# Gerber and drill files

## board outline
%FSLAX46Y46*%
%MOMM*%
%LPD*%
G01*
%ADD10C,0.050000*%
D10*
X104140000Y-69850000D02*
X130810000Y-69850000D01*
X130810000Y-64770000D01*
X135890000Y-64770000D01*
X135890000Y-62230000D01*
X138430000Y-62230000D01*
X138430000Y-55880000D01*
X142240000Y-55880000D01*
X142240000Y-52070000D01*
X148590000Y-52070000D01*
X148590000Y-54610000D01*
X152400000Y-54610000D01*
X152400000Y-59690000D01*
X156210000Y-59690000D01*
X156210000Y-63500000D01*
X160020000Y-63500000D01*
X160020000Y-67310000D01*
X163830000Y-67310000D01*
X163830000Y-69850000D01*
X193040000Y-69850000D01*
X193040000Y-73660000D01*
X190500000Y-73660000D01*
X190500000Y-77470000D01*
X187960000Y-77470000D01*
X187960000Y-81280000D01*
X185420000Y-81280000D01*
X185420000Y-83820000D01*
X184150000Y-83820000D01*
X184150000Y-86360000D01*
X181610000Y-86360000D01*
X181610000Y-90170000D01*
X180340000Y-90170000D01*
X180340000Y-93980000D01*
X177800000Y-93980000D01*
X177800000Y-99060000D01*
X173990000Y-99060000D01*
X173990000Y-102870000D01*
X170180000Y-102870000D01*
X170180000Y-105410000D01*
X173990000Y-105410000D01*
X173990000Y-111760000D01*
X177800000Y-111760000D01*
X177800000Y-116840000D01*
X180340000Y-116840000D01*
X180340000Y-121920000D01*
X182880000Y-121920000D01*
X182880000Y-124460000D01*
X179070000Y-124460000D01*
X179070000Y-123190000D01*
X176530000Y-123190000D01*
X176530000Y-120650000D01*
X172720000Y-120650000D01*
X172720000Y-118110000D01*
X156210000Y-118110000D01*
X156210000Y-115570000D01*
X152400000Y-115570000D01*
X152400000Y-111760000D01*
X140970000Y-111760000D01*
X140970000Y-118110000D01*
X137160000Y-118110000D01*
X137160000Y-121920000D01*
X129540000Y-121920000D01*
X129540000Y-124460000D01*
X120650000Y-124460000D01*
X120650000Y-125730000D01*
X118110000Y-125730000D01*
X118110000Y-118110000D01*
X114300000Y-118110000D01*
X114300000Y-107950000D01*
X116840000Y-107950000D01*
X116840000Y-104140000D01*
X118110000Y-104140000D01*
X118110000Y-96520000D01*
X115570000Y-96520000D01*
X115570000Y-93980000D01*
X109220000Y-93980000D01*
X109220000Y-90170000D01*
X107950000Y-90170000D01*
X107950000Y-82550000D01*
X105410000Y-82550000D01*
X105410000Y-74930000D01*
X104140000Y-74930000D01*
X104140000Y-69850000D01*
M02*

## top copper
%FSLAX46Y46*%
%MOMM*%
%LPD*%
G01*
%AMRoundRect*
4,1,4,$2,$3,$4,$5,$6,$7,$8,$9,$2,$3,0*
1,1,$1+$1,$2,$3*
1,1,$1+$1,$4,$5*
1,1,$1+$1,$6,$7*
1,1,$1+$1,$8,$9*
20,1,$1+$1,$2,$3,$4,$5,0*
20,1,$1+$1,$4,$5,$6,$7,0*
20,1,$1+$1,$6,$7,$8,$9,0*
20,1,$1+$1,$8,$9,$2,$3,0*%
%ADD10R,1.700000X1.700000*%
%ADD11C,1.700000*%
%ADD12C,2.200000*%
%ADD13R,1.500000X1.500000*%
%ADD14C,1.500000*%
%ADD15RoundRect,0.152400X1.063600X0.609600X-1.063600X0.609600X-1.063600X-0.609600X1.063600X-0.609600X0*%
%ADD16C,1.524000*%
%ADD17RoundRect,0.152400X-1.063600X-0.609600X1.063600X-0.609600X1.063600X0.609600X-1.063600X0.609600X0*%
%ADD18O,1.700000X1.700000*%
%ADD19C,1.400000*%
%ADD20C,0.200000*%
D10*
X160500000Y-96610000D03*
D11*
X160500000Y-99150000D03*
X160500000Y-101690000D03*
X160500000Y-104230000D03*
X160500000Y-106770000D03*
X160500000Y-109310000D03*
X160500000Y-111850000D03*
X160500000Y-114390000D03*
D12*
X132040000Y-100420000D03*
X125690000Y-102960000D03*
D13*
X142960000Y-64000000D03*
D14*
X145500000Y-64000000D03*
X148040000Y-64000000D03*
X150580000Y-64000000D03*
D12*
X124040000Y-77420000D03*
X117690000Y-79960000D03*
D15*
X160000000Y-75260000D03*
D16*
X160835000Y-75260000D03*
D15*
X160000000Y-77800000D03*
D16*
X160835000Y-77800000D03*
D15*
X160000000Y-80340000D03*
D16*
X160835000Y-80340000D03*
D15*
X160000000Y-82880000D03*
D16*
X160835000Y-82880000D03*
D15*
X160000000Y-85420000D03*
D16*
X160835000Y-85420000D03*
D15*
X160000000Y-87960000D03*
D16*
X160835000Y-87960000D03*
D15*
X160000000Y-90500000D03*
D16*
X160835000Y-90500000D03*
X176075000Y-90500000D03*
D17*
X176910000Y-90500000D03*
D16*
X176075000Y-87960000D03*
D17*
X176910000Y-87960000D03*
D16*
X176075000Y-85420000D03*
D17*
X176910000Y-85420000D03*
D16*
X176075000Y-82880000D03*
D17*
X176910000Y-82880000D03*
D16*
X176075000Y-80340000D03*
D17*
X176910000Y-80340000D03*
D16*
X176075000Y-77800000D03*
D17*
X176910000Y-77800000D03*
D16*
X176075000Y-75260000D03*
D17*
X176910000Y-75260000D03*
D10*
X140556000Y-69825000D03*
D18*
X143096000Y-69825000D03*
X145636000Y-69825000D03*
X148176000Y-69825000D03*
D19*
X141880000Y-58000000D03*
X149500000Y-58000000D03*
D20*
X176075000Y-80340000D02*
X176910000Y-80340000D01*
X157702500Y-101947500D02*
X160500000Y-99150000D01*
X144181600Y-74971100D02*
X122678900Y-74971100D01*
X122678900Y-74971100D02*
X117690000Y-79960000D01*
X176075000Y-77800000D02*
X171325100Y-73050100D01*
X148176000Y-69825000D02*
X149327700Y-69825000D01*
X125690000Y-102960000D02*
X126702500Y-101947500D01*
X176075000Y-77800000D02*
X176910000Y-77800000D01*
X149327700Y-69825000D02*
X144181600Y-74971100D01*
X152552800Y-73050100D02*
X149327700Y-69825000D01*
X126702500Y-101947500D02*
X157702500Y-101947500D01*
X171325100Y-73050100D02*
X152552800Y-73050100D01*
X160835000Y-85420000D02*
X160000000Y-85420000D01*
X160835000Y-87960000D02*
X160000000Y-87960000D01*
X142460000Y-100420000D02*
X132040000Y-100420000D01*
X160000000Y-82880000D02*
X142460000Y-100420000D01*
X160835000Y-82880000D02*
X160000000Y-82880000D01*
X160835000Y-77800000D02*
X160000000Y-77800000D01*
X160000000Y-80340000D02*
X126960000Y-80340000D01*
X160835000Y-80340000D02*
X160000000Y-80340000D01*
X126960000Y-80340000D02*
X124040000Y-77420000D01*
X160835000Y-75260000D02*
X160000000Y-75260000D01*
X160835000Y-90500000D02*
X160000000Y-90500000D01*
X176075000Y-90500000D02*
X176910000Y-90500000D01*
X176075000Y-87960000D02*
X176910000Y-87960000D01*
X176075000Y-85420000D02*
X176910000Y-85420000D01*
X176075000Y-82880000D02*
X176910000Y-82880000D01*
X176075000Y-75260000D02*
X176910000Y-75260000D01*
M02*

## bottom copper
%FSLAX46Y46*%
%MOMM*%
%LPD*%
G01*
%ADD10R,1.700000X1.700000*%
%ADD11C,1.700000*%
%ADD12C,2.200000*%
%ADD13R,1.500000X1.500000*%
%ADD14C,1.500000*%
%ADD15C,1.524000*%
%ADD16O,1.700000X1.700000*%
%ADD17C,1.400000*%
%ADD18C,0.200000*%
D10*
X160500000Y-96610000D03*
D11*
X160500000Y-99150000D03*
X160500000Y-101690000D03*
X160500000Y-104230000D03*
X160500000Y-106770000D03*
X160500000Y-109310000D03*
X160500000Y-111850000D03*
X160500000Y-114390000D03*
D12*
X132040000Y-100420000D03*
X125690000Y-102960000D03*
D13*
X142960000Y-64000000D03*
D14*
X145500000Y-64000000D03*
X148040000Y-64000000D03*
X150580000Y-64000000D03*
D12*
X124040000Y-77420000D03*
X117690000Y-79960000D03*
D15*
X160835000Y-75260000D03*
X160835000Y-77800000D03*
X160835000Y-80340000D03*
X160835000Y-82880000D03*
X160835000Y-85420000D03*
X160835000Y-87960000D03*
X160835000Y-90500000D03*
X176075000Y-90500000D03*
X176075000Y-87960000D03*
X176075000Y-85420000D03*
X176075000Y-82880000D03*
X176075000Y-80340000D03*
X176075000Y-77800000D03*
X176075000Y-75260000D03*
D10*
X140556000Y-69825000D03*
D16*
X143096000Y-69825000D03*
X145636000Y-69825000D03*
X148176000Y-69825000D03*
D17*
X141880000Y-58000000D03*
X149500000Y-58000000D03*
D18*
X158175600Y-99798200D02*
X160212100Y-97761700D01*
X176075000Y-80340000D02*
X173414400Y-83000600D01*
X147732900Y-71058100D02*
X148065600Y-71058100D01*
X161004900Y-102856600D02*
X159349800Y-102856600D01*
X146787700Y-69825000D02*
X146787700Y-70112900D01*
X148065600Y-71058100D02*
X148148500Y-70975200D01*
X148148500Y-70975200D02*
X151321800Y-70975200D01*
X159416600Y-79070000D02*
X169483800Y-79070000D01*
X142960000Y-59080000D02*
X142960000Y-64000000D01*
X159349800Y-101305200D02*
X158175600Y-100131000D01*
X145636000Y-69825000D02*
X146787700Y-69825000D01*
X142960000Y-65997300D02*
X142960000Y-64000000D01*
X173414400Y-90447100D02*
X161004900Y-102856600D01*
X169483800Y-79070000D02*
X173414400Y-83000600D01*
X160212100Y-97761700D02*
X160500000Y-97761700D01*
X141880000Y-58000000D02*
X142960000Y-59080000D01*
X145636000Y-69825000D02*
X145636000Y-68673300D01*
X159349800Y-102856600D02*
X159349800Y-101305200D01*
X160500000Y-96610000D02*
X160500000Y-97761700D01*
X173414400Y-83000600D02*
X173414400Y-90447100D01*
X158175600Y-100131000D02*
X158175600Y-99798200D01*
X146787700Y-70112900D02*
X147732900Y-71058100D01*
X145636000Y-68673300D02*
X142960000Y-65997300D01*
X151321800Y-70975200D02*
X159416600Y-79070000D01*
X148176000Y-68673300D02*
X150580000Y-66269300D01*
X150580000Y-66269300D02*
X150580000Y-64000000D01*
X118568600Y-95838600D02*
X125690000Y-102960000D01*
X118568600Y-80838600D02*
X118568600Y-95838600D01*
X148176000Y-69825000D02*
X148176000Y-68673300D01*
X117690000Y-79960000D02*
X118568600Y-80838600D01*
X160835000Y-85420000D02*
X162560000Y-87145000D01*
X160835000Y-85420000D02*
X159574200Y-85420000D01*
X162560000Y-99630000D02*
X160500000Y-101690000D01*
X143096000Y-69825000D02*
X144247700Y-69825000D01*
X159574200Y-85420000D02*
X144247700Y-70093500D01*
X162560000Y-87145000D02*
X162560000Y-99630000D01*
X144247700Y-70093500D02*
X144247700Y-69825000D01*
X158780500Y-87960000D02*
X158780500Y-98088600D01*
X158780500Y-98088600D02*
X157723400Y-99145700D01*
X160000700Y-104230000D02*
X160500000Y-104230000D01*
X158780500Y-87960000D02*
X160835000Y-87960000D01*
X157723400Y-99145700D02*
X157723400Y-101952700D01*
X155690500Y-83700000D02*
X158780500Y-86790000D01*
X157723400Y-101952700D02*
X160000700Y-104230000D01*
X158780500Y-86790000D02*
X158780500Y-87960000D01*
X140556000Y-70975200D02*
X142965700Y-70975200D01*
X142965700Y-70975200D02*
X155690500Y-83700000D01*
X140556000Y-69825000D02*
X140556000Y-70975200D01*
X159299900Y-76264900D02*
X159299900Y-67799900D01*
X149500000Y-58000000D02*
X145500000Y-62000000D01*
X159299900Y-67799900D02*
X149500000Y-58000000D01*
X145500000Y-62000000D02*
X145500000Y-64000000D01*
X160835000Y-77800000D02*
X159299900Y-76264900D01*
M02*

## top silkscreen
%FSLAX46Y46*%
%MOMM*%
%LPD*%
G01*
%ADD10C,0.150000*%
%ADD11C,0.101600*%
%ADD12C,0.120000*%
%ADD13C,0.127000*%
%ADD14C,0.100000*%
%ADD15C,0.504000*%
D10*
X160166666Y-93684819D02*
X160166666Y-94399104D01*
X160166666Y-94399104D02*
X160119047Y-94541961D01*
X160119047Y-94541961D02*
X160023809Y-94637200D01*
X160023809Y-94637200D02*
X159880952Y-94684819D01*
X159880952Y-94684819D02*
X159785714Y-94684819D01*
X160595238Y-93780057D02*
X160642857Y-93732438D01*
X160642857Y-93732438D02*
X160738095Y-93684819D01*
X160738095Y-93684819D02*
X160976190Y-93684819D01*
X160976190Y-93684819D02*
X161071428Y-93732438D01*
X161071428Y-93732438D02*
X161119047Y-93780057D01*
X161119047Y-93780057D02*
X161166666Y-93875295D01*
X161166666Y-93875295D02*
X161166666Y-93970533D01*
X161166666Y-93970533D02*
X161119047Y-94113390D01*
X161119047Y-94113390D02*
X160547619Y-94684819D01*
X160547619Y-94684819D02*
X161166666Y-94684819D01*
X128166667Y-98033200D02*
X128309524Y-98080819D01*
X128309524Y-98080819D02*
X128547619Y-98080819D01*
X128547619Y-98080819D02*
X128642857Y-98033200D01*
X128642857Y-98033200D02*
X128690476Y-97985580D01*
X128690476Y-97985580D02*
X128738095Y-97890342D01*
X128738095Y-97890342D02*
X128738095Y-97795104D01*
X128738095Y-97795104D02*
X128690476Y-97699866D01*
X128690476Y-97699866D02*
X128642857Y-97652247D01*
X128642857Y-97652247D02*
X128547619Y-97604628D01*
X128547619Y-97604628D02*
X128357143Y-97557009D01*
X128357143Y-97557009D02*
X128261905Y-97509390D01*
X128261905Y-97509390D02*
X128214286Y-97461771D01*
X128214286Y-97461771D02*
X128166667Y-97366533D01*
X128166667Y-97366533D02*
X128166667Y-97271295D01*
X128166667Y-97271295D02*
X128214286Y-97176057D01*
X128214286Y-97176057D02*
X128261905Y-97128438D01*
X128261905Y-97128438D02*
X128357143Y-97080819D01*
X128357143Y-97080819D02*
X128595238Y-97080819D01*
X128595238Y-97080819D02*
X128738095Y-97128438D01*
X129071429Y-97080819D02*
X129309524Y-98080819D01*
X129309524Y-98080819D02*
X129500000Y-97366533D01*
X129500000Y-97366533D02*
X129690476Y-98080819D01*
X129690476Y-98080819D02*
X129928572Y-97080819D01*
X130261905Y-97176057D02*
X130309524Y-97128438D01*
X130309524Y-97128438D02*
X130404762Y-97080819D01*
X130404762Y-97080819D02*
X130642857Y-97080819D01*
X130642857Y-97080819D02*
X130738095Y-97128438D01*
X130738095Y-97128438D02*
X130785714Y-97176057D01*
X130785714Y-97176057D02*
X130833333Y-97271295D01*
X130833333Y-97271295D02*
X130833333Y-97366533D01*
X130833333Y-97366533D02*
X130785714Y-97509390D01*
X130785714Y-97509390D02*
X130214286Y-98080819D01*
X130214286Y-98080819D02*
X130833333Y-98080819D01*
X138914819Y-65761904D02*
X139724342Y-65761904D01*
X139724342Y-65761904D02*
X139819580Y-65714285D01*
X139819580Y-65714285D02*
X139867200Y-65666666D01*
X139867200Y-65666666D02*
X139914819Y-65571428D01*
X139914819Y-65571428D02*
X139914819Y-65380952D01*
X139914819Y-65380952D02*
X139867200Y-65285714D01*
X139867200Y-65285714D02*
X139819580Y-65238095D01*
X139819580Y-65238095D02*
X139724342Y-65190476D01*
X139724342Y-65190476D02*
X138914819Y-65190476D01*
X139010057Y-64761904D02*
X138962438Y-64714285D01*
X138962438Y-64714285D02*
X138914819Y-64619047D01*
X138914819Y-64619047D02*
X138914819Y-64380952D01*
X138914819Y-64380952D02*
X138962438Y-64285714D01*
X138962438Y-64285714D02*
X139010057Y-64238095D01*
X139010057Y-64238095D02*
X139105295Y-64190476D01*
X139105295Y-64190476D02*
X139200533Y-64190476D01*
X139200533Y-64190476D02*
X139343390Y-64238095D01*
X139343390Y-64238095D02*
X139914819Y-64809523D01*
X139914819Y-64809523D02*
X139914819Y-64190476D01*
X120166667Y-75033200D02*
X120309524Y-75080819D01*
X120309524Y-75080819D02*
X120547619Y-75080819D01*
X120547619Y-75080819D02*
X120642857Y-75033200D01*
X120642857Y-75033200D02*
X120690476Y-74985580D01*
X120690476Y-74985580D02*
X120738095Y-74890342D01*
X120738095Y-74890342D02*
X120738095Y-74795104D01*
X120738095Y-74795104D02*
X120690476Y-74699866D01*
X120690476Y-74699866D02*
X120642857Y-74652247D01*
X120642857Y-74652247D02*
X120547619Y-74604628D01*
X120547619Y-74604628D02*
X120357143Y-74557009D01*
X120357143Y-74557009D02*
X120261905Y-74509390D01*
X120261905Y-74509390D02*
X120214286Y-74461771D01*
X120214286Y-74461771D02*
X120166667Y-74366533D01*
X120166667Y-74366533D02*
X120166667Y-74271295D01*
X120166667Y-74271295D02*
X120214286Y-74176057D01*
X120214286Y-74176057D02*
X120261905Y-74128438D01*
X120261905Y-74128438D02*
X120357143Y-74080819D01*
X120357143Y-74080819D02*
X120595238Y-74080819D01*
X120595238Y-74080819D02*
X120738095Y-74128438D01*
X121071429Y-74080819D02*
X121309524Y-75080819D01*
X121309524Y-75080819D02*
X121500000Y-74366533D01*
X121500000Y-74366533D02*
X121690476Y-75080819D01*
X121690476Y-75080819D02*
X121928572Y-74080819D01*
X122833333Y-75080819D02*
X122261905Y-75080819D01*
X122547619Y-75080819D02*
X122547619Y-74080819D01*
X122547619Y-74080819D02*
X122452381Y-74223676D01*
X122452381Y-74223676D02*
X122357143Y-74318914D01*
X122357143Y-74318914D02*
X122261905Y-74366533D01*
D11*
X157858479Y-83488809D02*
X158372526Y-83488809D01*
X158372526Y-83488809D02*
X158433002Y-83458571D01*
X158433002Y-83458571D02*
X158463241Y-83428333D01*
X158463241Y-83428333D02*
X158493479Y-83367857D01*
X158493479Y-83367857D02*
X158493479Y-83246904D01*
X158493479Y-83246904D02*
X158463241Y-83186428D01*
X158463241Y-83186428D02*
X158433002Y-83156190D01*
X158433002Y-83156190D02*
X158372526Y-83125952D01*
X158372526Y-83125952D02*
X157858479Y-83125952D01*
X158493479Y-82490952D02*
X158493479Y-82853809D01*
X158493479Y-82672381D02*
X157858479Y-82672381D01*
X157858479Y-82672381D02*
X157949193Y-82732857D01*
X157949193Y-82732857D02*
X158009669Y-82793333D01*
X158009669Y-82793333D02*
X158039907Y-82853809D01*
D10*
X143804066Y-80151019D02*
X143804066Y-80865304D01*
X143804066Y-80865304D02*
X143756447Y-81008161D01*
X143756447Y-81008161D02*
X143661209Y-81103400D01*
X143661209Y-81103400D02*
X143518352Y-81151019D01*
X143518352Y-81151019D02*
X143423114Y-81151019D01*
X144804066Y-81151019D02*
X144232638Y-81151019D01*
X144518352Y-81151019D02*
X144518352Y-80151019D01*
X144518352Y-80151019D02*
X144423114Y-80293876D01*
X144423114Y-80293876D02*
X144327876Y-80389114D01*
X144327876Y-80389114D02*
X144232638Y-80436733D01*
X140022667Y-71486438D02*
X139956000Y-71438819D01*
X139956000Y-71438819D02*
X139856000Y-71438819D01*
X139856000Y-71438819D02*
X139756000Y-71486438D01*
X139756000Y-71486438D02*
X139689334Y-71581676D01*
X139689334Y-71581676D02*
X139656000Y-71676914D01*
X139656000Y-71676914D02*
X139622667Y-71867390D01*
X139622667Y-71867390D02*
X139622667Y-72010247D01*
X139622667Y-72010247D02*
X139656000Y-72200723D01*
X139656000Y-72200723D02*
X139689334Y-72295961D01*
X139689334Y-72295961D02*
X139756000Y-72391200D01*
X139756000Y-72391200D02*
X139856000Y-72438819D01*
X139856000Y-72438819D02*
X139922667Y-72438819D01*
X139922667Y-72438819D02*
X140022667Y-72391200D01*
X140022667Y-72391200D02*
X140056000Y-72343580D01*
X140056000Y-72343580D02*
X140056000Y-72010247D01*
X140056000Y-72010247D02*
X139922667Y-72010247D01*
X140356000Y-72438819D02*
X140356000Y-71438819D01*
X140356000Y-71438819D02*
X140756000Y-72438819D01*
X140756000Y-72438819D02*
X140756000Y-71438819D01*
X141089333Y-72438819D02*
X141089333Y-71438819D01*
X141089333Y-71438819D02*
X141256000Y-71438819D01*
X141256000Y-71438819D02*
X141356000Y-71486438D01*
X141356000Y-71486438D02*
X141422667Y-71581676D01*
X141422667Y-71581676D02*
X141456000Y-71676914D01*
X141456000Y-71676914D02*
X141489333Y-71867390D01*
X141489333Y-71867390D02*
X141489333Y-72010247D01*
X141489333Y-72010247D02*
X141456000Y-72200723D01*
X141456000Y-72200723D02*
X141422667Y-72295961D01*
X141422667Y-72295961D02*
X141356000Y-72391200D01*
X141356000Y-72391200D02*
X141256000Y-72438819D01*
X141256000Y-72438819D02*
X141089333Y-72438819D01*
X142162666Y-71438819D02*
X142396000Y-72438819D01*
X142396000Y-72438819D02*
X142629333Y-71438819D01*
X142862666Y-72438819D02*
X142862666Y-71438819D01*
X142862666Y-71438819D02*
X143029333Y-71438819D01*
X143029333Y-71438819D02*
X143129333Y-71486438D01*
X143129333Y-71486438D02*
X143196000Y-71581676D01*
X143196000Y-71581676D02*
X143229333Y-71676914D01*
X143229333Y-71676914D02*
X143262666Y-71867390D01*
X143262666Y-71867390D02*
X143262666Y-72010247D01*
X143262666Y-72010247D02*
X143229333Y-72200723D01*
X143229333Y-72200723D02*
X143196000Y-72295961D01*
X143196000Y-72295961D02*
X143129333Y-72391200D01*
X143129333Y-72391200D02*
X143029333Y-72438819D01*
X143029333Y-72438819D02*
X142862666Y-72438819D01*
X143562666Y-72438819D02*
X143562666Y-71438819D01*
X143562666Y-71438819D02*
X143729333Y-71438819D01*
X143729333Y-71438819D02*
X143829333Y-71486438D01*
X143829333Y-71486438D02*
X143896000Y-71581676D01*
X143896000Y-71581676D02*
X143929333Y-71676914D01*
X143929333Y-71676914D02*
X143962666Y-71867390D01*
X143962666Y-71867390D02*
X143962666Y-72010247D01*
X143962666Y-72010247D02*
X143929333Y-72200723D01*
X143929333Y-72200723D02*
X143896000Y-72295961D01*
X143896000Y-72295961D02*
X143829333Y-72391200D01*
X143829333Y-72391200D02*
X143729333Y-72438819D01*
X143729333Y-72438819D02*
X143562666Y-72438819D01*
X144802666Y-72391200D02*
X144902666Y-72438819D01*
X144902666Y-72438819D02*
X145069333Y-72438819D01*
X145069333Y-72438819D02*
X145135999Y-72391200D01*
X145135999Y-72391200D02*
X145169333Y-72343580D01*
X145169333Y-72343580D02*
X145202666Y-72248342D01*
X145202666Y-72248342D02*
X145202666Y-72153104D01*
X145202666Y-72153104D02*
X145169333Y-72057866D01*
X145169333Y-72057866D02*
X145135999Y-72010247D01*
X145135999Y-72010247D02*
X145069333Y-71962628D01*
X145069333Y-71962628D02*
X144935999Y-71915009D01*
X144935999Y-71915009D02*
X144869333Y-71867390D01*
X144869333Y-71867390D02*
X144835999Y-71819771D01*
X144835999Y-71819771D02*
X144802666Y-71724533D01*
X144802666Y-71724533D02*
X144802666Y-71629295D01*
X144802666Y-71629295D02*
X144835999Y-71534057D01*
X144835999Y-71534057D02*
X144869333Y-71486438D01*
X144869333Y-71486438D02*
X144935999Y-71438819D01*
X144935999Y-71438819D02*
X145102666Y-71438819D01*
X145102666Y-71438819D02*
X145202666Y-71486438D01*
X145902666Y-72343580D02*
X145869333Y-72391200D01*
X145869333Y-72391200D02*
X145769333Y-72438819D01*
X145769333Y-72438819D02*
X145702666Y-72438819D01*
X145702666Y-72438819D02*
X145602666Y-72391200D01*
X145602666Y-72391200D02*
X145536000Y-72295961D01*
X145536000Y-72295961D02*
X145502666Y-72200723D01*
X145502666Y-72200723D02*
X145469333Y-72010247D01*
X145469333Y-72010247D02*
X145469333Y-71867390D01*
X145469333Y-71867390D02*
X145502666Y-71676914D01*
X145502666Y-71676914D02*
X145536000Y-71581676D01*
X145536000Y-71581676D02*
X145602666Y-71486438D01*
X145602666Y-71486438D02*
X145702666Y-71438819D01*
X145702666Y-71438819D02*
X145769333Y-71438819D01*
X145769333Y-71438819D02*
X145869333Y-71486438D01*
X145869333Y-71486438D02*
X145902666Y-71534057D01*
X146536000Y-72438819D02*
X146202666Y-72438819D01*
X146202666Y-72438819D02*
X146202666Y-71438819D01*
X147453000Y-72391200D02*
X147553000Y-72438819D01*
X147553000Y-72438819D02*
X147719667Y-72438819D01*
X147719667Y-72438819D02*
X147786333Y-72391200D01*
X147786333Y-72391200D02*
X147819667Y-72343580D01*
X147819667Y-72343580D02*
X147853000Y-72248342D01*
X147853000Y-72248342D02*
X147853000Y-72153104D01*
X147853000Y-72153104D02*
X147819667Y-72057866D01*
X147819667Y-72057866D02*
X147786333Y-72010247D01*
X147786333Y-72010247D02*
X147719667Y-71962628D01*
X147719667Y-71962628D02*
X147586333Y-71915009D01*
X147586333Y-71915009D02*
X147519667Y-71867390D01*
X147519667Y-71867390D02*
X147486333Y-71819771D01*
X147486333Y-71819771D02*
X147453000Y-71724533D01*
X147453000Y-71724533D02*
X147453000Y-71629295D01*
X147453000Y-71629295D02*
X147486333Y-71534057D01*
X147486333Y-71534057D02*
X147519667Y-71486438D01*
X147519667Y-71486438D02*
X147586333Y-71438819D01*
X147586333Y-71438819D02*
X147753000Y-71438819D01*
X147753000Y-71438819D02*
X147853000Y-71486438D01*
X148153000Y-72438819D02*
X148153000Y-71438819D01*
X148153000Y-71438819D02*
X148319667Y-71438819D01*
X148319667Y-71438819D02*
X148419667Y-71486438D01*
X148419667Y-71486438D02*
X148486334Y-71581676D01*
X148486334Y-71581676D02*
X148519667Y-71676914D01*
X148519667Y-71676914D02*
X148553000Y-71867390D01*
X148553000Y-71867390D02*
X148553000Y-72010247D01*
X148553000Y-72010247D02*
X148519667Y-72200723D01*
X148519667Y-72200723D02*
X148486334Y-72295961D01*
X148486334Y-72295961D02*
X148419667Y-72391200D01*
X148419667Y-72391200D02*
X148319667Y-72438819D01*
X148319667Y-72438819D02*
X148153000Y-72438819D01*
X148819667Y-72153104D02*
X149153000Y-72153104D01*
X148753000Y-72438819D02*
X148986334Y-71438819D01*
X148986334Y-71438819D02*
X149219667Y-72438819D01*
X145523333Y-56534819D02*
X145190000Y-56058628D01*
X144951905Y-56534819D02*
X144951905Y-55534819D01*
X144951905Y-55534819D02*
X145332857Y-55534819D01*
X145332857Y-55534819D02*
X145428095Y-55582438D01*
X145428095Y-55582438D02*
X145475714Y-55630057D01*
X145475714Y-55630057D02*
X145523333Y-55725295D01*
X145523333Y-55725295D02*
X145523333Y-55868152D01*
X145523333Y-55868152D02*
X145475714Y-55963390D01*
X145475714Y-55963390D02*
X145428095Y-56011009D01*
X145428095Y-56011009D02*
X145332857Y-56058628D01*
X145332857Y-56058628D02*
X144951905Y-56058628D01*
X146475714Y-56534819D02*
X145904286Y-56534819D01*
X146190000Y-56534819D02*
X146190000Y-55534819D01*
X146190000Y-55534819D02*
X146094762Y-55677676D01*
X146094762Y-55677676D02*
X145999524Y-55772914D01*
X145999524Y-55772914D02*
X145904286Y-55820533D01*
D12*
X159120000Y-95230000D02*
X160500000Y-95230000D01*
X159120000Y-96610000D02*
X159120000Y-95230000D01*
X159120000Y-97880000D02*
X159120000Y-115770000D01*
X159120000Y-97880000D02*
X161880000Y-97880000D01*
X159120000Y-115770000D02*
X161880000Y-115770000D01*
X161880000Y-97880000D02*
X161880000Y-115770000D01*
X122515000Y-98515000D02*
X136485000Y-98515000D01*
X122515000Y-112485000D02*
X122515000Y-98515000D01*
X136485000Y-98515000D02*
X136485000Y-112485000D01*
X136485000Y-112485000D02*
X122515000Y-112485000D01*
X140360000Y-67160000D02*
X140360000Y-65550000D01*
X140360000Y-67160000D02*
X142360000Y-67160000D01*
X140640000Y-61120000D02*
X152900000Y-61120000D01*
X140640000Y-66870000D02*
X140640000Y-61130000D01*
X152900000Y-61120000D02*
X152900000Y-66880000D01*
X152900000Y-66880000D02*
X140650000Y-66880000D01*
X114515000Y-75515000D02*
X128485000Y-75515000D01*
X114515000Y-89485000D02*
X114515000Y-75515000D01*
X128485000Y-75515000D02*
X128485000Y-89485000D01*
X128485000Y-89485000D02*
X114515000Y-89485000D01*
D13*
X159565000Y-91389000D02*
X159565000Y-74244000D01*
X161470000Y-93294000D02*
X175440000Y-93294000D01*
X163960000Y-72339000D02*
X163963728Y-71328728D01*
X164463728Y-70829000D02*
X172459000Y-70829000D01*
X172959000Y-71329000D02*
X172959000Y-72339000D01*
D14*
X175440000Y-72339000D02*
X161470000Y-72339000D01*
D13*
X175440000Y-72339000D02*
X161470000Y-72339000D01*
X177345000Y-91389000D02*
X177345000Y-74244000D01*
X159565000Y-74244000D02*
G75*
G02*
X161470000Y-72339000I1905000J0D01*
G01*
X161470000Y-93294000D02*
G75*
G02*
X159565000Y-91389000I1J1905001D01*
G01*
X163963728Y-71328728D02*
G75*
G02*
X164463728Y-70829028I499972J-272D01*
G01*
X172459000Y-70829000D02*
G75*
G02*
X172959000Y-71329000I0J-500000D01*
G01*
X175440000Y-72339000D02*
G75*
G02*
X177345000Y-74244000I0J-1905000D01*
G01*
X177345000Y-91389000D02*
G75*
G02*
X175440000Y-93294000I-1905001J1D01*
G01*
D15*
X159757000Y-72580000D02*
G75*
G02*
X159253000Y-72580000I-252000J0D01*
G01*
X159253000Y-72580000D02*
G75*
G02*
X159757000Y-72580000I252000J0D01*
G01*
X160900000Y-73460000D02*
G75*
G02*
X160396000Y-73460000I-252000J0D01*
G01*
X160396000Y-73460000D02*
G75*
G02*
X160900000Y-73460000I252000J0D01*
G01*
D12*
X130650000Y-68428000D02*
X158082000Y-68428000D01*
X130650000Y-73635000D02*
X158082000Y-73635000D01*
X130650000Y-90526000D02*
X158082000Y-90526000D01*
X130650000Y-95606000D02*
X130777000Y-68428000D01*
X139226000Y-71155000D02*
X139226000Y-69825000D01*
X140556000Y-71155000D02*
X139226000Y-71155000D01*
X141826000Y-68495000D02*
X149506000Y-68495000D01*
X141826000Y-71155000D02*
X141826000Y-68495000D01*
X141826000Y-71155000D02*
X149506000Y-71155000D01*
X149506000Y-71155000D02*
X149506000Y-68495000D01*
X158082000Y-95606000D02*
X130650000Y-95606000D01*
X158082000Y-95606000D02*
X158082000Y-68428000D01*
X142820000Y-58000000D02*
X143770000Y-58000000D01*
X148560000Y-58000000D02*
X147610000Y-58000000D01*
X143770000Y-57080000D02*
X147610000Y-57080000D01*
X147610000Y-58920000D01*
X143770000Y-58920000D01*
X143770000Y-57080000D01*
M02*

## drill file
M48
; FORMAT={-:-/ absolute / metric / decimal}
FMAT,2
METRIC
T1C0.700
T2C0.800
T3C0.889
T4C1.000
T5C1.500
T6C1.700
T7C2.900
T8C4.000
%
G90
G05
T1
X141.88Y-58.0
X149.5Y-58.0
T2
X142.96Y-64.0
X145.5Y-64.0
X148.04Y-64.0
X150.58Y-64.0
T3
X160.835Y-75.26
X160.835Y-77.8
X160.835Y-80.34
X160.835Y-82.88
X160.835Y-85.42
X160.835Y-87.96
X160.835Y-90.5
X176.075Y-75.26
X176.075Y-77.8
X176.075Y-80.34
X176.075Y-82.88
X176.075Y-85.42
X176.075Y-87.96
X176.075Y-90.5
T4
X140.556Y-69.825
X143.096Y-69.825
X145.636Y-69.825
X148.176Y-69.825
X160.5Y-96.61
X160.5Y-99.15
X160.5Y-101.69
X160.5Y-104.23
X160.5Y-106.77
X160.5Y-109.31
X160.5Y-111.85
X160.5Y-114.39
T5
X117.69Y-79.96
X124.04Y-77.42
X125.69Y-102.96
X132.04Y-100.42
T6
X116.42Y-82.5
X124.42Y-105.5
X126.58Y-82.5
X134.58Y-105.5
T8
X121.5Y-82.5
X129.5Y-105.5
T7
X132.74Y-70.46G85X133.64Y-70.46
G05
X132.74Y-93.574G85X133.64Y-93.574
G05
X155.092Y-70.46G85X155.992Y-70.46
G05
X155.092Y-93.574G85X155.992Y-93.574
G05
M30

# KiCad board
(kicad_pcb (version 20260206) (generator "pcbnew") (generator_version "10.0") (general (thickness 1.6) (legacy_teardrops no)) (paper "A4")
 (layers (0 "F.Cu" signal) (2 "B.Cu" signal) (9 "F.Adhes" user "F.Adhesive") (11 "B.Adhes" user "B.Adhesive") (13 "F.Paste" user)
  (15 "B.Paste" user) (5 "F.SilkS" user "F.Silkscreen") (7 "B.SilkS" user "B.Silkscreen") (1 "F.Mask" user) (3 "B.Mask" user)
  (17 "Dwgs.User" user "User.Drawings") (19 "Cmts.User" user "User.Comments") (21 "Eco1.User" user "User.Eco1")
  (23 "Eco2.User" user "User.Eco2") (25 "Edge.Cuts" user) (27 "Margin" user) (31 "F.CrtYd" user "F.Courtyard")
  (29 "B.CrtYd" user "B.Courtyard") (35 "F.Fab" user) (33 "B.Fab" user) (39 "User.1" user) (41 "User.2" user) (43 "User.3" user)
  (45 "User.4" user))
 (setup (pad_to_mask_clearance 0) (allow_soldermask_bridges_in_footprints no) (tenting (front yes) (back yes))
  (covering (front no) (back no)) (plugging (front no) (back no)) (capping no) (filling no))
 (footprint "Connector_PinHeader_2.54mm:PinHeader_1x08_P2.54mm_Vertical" (layer "F.Cu") (at 160.5 96.61)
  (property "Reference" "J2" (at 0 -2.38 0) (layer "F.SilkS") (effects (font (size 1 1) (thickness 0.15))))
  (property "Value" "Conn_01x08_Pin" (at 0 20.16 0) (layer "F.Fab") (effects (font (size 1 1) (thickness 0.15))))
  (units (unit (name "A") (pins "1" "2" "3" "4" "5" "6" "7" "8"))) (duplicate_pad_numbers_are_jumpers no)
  (fp_line (start -1.38 -1.38) (end 0 -1.38) (stroke (width 0.12) (type solid)) (layer "F.SilkS"))
  (fp_line (start -1.38 0) (end -1.38 -1.38) (stroke (width 0.12) (type solid)) (layer "F.SilkS"))
  (fp_line (start -1.38 1.27) (end -1.38 19.16) (stroke (width 0.12) (type solid)) (layer "F.SilkS"))
  (fp_line (start -1.38 1.27) (end 1.38 1.27) (stroke (width 0.12) (type solid)) (layer "F.SilkS"))
  (fp_line (start -1.38 19.16) (end 1.38 19.16) (stroke (width 0.12) (type solid)) (layer "F.SilkS"))
  (fp_line (start 1.38 1.27) (end 1.38 19.16) (stroke (width 0.12) (type solid)) (layer "F.SilkS"))
  (pad "1" thru_hole rect (at 0 0) (size 1.7 1.7) (drill 1) (layers "*.Cu" "*.Mask") (remove_unused_layers no) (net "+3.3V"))
  (pad "2" thru_hole circle (at 0 2.54) (size 1.7 1.7) (drill 1) (layers "*.Cu" "*.Mask") (remove_unused_layers no) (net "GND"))
  (pad "3" thru_hole circle (at 0 5.08) (size 1.7 1.7) (drill 1) (layers "*.Cu" "*.Mask") (remove_unused_layers no) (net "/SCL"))
  (pad "4" thru_hole circle (at 0 7.62) (size 1.7 1.7) (drill 1) (layers "*.Cu" "*.Mask") (remove_unused_layers no) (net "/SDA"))
  (pad "5" thru_hole circle (at 0 10.16) (size 1.7 1.7) (drill 1) (layers "*.Cu" "*.Mask") (remove_unused_layers no)
   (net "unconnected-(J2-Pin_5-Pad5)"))
  (pad "6" thru_hole circle (at 0 12.7) (size 1.7 1.7) (drill 1) (layers "*.Cu" "*.Mask") (remove_unused_layers no)
   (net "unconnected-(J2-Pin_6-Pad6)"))
  (pad "7" thru_hole circle (at 0 15.24) (size 1.7 1.7) (drill 1) (layers "*.Cu" "*.Mask") (remove_unused_layers no)
   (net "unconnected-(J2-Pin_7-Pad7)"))
  (pad "8" thru_hole circle (at 0 17.78) (size 1.7 1.7) (drill 1) (layers "*.Cu" "*.Mask") (remove_unused_layers no)
   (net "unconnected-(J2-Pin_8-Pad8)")))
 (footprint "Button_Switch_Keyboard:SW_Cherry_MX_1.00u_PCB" (layer "F.Cu") (at 132.04 100.42)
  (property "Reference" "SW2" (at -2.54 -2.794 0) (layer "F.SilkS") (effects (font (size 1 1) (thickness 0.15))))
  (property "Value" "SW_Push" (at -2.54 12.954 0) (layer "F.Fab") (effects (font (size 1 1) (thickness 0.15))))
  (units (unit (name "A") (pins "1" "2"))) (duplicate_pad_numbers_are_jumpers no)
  (fp_line (start -9.525 -1.905) (end 4.445 -1.905) (stroke (width 0.12) (type solid)) (layer "F.SilkS"))
  (fp_line (start -9.525 12.065) (end -9.525 -1.905) (stroke (width 0.12) (type solid)) (layer "F.SilkS"))
  (fp_line (start 4.445 -1.905) (end 4.445 12.065) (stroke (width 0.12) (type solid)) (layer "F.SilkS"))
  (fp_line (start 4.445 12.065) (end -9.525 12.065) (stroke (width 0.12) (type solid)) (layer "F.SilkS"))
  (pad "" np_thru_hole circle (at -7.62 5.08) (size 1.7 1.7) (drill 1.7) (layers "*.Cu" "*.Mask"))
  (pad "" np_thru_hole circle (at -2.54 5.08) (size 4 4) (drill 4) (layers "*.Cu" "*.Mask"))
  (pad "" np_thru_hole circle (at 2.54 5.08) (size 1.7 1.7) (drill 1.7) (layers "*.Cu" "*.Mask"))
  (pad "1" thru_hole circle (at 0 0) (size 2.2 2.2) (drill 1.5) (layers "*.Cu" "*.Mask") (remove_unused_layers no) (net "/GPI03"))
  (pad "2" thru_hole circle (at -6.35 2.54) (size 2.2 2.2) (drill 1.5) (layers "*.Cu" "*.Mask") (remove_unused_layers no) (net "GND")))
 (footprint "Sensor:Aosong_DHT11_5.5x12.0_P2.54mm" (layer "F.Cu") (at 142.96 64 90)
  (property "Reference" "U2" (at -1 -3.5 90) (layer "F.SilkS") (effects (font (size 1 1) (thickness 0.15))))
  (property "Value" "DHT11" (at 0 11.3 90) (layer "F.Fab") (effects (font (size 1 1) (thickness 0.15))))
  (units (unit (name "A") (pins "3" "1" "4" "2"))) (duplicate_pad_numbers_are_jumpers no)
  (fp_line (start -3.16 -2.6) (end -1.55 -2.6) (stroke (width 0.12) (type solid)) (layer "F.SilkS"))
  (fp_line (start -3.16 -2.6) (end -3.16 -0.6) (stroke (width 0.12) (type solid)) (layer "F.SilkS"))
  (fp_line (start 2.88 -2.32) (end 2.88 9.94) (stroke (width 0.12) (type solid)) (layer "F.SilkS"))
  (fp_line (start -2.87 -2.32) (end 2.87 -2.32) (stroke (width 0.12) (type solid)) (layer "F.SilkS"))
  (fp_line (start 2.88 9.94) (end -2.88 9.94) (stroke (width 0.12) (type solid)) (layer "F.SilkS"))
  (fp_line (start -2.88 9.94) (end -2.88 -2.31) (stroke (width 0.12) (type solid)) (layer "F.SilkS"))
  (pad "1" thru_hole rect (at 0 0 90) (size 1.5 1.5) (drill 0.8) (layers "*.Cu" "*.Mask") (remove_unused_layers no) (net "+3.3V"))
  (pad "2" thru_hole circle (at 0 2.54 90) (size 1.5 1.5) (drill 0.8) (layers "*.Cu" "*.Mask") (remove_unused_layers no) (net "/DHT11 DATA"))
  (pad "3" thru_hole circle (at 0 5.08 90) (size 1.5 1.5) (drill 0.8) (layers "*.Cu" "*.Mask") (remove_unused_layers no)
   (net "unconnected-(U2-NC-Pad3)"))
  (pad "4" thru_hole circle (at 0 7.62 90) (size 1.5 1.5) (drill 0.8) (layers "*.Cu" "*.Mask") (remove_unused_layers no) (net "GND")))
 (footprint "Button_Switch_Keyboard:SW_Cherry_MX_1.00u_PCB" (layer "F.Cu") (at 124.04 77.42)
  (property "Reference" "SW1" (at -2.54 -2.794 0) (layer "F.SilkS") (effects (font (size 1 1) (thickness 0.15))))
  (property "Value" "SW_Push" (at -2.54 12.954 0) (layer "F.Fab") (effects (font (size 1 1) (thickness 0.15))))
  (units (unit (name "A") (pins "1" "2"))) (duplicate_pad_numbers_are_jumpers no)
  (fp_line (start -9.525 -1.905) (end 4.445 -1.905) (stroke (width 0.12) (type solid)) (layer "F.SilkS"))
  (fp_line (start -9.525 12.065) (end -9.525 -1.905) (stroke (width 0.12) (type solid)) (layer "F.SilkS"))
  (fp_line (start 4.445 -1.905) (end 4.445 12.065) (stroke (width 0.12) (type solid)) (layer "F.SilkS"))
  (fp_line (start 4.445 12.065) (end -9.525 12.065) (stroke (width 0.12) (type solid)) (layer "F.SilkS"))
  (pad "" np_thru_hole circle (at -7.62 5.08) (size 1.7 1.7) (drill 1.7) (layers "*.Cu" "*.Mask"))
  (pad "" np_thru_hole circle (at -2.54 5.08) (size 4 4) (drill 4) (layers "*.Cu" "*.Mask"))
  (pad "" np_thru_hole circle (at 2.54 5.08) (size 1.7 1.7) (drill 1.7) (layers "*.Cu" "*.Mask"))
  (pad "1" thru_hole circle (at 0 0) (size 2.2 2.2) (drill 1.5) (layers "*.Cu" "*.Mask") (remove_unused_layers no) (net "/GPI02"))
  (pad "2" thru_hole circle (at -6.35 2.54) (size 2.2 2.2) (drill 1.5) (layers "*.Cu" "*.Mask") (remove_unused_layers no) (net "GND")))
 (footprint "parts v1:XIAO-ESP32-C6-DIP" (layer "F.Cu") (at 168.455 82.88 90)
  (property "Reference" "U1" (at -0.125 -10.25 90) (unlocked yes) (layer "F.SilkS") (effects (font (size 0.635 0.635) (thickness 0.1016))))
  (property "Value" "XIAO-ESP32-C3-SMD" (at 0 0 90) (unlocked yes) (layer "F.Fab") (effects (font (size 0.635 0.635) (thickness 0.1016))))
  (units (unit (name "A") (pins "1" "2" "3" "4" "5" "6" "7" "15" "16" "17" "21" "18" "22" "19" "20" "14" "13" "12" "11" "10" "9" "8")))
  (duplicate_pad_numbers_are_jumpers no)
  (fp_line (start -8.509 -8.89) (end 8.636 -8.89) (stroke (width 0.127) (type solid)) (layer "F.SilkS"))
  (fp_line (start -10.414 -6.985) (end -10.414 6.985) (stroke (width 0.127) (type solid)) (layer "F.SilkS"))
  (fp_line (start 10.541 -4.495) (end 11.551272 -4.491272) (stroke (width 0.127) (type solid)) (layer "F.SilkS"))
  (fp_line (start 12.051 -3.991272) (end 12.051 4.004) (stroke (width 0.127) (type solid)) (layer "F.SilkS"))
  (fp_line (start 11.551 4.504) (end 10.541 4.504) (stroke (width 0.127) (type solid)) (layer "F.SilkS"))
  (fp_line (start 10.541 6.985) (end 10.541 -6.985) (stroke (width 0.1) (type solid)) (layer "F.SilkS"))
  (fp_line (start 10.541 6.985) (end 10.541 -6.985) (stroke (width 0.127) (type solid)) (layer "F.SilkS"))
  (fp_line (start -8.509 8.89) (end 8.636 8.89) (stroke (width 0.127) (type solid)) (layer "F.SilkS"))
  (fp_arc (start 8.636 -8.89) (mid 9.983038 -8.332038) (end 10.541 -6.985) (stroke (width 0.127) (type solid)) (layer "F.SilkS"))
  (fp_arc (start -10.414 -6.985) (mid -9.856038 -8.332038) (end -8.509 -8.89) (stroke (width 0.127) (type solid)) (layer "F.SilkS"))
  (fp_arc (start 11.551272 -4.491272) (mid 11.904644 -4.344724) (end 12.051 -3.991272) (stroke (width 0.127) (type default))
   (layer "F.SilkS"))
  (fp_arc (start 12.051 4.004) (mid 11.904553 4.357553) (end 11.551 4.504) (stroke (width 0.127) (type default)) (layer "F.SilkS"))
  (fp_arc (start 10.541 6.985) (mid 9.983038 8.332038) (end 8.636 8.89) (stroke (width 0.127) (type solid)) (layer "F.SilkS"))
  (fp_arc (start -8.509 8.89) (mid -9.856038 8.332038) (end -10.414 6.985) (stroke (width 0.127) (type solid)) (layer "F.SilkS"))
  (fp_circle (center 10.3 -8.95) (end 10.554 -8.95) (stroke (width 0.5) (type solid)) (fill yes) (layer "F.SilkS"))
  (fp_circle (center 9.42 -7.807) (end 9.674 -7.807) (stroke (width 0.5) (type solid)) (fill yes) (layer "F.SilkS"))
  (pad "1" smd roundrect (at 7.62 -8.455 180) (size 2.432 1.524) (layers "F.Cu" "F.Mask") (roundrect_rratio 0.1)
   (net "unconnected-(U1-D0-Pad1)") (thermal_bridge_angle 45))
  (pad "1" thru_hole circle (at 7.62 -7.62 180) (size 1.524 1.524) (drill 0.889) (layers "*.Cu" "*.Mask") (remove_unused_layers no)
   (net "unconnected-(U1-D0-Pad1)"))
  (pad "2" smd roundrect (at 5.08 -8.455 180) (size 2.432 1.524) (layers "F.Cu" "F.Mask") (roundrect_rratio 0.1) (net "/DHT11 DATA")
   (thermal_bridge_angle 45))
  (pad "2" thru_hole circle (at 5.08 -7.62 180) (size 1.524 1.524) (drill 0.889) (layers "*.Cu" "*.Mask") (remove_unused_layers no)
   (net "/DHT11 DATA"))
  (pad "3" smd roundrect (at 2.54 -8.455 180) (size 2.432 1.524) (layers "F.Cu" "F.Mask") (roundrect_rratio 0.1) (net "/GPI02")
   (thermal_bridge_angle 45))
  (pad "3" thru_hole circle (at 2.54 -7.62 180) (size 1.524 1.524) (drill 0.889) (layers "*.Cu" "*.Mask") (remove_unused_layers no)
   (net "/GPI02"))
  (pad "4" smd roundrect (at 0 -8.455 180) (size 2.432 1.524) (layers "F.Cu" "F.Mask") (roundrect_rratio 0.1) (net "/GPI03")
   (thermal_bridge_angle 45))
  (pad "4" thru_hole circle (at 0 -7.62 180) (size 1.524 1.524) (drill 0.889) (layers "*.Cu" "*.Mask") (remove_unused_layers no)
   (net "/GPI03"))
  (pad "5" smd roundrect (at -2.54 -8.455 180) (size 2.432 1.524) (layers "F.Cu" "F.Mask") (roundrect_rratio 0.1) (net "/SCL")
   (thermal_bridge_angle 45))
  (pad "5" thru_hole circle (at -2.54 -7.62 180) (size 1.524 1.524) (drill 0.889) (layers "*.Cu" "*.Mask") (remove_unused_layers no)
   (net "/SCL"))
  (pad "6" smd roundrect (at -5.08 -8.455 180) (size 2.432 1.524) (layers "F.Cu" "F.Mask") (roundrect_rratio 0.1) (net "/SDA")
   (thermal_bridge_angle 45))
  (pad "6" thru_hole circle (at -5.08 -7.62 180) (size 1.524 1.524) (drill 0.889) (layers "*.Cu" "*.Mask") (remove_unused_layers no)
   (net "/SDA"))
  (pad "7" smd roundrect (at -7.62 -8.455 180) (size 2.432 1.524) (layers "F.Cu" "F.Mask") (roundrect_rratio 0.1)
   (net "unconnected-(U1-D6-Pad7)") (thermal_bridge_angle 45))
  (pad "7" thru_hole circle (at -7.62 -7.62 180) (size 1.524 1.524) (drill 0.889) (layers "*.Cu" "*.Mask") (remove_unused_layers no)
   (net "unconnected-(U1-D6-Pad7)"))
  (pad "8" thru_hole circle (at -7.62 7.62) (size 1.524 1.524) (drill 0.889) (layers "*.Cu" "*.Mask") (remove_unused_layers no)
   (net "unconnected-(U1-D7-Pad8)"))
  (pad "8" smd roundrect (at -7.62 8.455) (size 2.432 1.524) (layers "F.Cu" "F.Mask") (roundrect_rratio 0.1)
   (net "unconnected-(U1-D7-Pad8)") (thermal_bridge_angle 45))
  (pad "9" thru_hole circle (at -5.08 7.62) (size 1.524 1.524) (drill 0.889) (layers "*.Cu" "*.Mask") (remove_unused_layers no)
   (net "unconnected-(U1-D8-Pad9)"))
  (pad "9" smd roundrect (at -5.08 8.455) (size 2.432 1.524) (layers "F.Cu" "F.Mask") (roundrect_rratio 0.1)
   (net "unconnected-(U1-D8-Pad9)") (thermal_bridge_angle 45))
  (pad "10" thru_hole circle (at -2.54 7.62) (size 1.524 1.524) (drill 0.889) (layers "*.Cu" "*.Mask") (remove_unused_layers no)
   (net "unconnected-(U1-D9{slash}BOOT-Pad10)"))
  (pad "10" smd roundrect (at -2.54 8.455) (size 2.432 1.524) (layers "F.Cu" "F.Mask") (roundrect_rratio 0.1)
   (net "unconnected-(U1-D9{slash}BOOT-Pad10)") (thermal_bridge_angle 45))
  (pad "11" thru_hole circle (at 0 7.62) (size 1.524 1.524) (drill 0.889) (layers "*.Cu" "*.Mask") (remove_unused_layers no)
   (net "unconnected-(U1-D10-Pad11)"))
  (pad "11" smd roundrect (at 0 8.455) (size 2.432 1.524) (layers "F.Cu" "F.Mask") (roundrect_rratio 0.1) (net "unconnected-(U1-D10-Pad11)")
   (thermal_bridge_angle 45))
  (pad "12" thru_hole circle (at 2.54 7.62) (size 1.524 1.524) (drill 0.889) (layers "*.Cu" "*.Mask") (remove_unused_layers no)
   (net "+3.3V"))
  (pad "12" smd roundrect (at 2.54 8.455) (size 2.432 1.524) (layers "F.Cu" "F.Mask") (roundrect_rratio 0.1) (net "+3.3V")
   (thermal_bridge_angle 45))
  (pad "13" thru_hole circle (at 5.08 7.62) (size 1.524 1.524) (drill 0.889) (layers "*.Cu" "*.Mask") (remove_unused_layers no) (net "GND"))
  (pad "13" smd roundrect (at 5.08 8.455) (size 2.432 1.524) (layers "F.Cu" "F.Mask") (roundrect_rratio 0.1) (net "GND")
   (thermal_bridge_angle 45))
  (pad "14" thru_hole circle (at 7.62 7.62) (size 1.524 1.524) (drill 0.889) (layers "*.Cu" "*.Mask") (remove_unused_layers no) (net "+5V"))
  (pad "14" smd roundrect (at 7.62 8.455) (size 2.432 1.524) (layers "F.Cu" "F.Mask") (roundrect_rratio 0.1) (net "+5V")
   (thermal_bridge_angle 45)))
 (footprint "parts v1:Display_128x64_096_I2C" (layer "F.Cu") (at 144.366 69.825)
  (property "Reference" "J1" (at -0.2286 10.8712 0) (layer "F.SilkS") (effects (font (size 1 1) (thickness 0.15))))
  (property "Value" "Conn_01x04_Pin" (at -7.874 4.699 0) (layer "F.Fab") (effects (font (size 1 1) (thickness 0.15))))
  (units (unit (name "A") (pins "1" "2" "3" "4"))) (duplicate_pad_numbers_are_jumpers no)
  (fp_line (start -13.716 -1.397) (end 13.716 -1.397) (stroke (width 0.12) (type solid)) (layer "F.SilkS"))
  (fp_line (start -13.716 3.81) (end 13.716 3.81) (stroke (width 0.12) (type solid)) (layer "F.SilkS"))
  (fp_line (start -13.716 20.701) (end 13.716 20.701) (stroke (width 0.12) (type solid)) (layer "F.SilkS"))
  (fp_line (start -13.716 25.781) (end -13.589 -1.397) (stroke (width 0.12) (type solid)) (layer "F.SilkS"))
  (fp_line (start -5.14 1.33) (end -5.14 0) (stroke (width 0.12) (type solid)) (layer "F.SilkS"))
  (fp_line (start -3.81 1.33) (end -5.14 1.33) (stroke (width 0.12) (type solid)) (layer "F.SilkS"))
  (fp_line (start -2.54 -1.33) (end 5.14 -1.33) (stroke (width 0.12) (type solid)) (layer "F.SilkS"))
  (fp_line (start -2.54 1.33) (end -2.54 -1.33) (stroke (width 0.12) (type solid)) (layer "F.SilkS"))
  (fp_line (start -2.54 1.33) (end 5.14 1.33) (stroke (width 0.12) (type solid)) (layer "F.SilkS"))
  (fp_line (start 5.14 1.33) (end 5.14 -1.33) (stroke (width 0.12) (type solid)) (layer "F.SilkS"))
  (fp_line (start 13.716 25.781) (end -13.716 25.781) (stroke (width 0.12) (type solid)) (layer "F.SilkS"))
  (fp_line (start 13.716 25.781) (end 13.716 -1.397) (stroke (width 0.12) (type solid)) (layer "F.SilkS"))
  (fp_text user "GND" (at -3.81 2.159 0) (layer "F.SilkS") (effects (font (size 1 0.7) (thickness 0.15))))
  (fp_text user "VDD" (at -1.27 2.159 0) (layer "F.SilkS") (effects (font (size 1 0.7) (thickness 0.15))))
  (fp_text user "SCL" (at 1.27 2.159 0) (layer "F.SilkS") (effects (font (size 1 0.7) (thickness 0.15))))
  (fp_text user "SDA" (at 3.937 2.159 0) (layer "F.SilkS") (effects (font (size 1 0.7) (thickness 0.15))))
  (pad "" np_thru_hole oval (at -11.176 0.635) (size 3.8 2.9) (drill oval 3.8 2.9) (layers "*.Cu" "*.Mask"))
  (pad "" np_thru_hole oval (at -11.176 23.749) (size 3.8 2.9) (drill oval 3.8 2.9) (layers "*.Cu" "*.Mask"))
  (pad "" np_thru_hole oval (at 11.176 0.635) (size 3.8 2.9) (drill oval 3.8 2.9) (layers "*.Cu" "*.Mask"))
  (pad "" np_thru_hole oval (at 11.176 23.749) (size 3.8 2.9) (drill oval 3.8 2.9) (layers "*.Cu" "*.Mask"))
  (pad "1" thru_hole rect (at -3.81 0 90) (size 1.7 1.7) (drill 1) (layers "*.Cu" "*.Mask") (remove_unused_layers no) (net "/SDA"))
  (pad "2" thru_hole oval (at -1.27 0 90) (size 1.7 1.7) (drill 1) (layers "*.Cu" "*.Mask") (remove_unused_layers no) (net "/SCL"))
  (pad "3" thru_hole oval (at 1.27 0 90) (size 1.7 1.7) (drill 1) (layers "*.Cu" "*.Mask") (remove_unused_layers no) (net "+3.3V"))
  (pad "4" thru_hole oval (at 3.81 0 90) (size 1.7 1.7) (drill 1) (layers "*.Cu" "*.Mask") (remove_unused_layers no) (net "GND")))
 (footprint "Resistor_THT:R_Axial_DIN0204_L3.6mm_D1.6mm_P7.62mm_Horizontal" (layer "F.Cu") (at 141.88 58)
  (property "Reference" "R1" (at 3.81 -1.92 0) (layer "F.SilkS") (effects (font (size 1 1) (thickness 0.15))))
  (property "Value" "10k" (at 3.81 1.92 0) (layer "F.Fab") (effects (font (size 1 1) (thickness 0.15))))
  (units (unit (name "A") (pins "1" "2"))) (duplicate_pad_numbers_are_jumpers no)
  (fp_line (start 0.94 0) (end 1.89 0) (stroke (width 0.12) (type solid)) (layer "F.SilkS"))
  (fp_line (start 6.68 0) (end 5.73 0) (stroke (width 0.12) (type solid)) (layer "F.SilkS"))
  (fp_rect (start 1.89 -0.92) (end 5.73 0.92) (stroke (width 0.12) (type solid)) (fill no) (layer "F.SilkS"))
  (pad "1" thru_hole circle (at 0 0) (size 1.4 1.4) (drill 0.7) (layers "*.Cu" "*.Mask") (remove_unused_layers no) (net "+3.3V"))
  (pad "2" thru_hole circle (at 7.62 0) (size 1.4 1.4) (drill 0.7) (layers "*.Cu" "*.Mask") (remove_unused_layers no) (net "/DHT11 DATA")))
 (gr_poly
  (pts (xy 104.14 69.85) (xy 130.81 69.85) (xy 130.81 64.77) (xy 135.89 64.77) (xy 135.89 62.23) (xy 138.43 62.23) (xy 138.43 55.88)
   (xy 142.24 55.88) (xy 142.24 52.07) (xy 148.59 52.07) (xy 148.59 54.61) (xy 152.4 54.61) (xy 152.4 59.69) (xy 156.21 59.69)
   (xy 156.21 63.5) (xy 160.02 63.5) (xy 160.02 67.31) (xy 163.83 67.31) (xy 163.83 69.85) (xy 193.04 69.85) (xy 193.04 73.66)
   (xy 190.5 73.66) (xy 190.5 77.47) (xy 187.96 77.47) (xy 187.96 81.28) (xy 185.42 81.28) (xy 185.42 83.82) (xy 184.15 83.82)
   (xy 184.15 86.36) (xy 181.61 86.36) (xy 181.61 90.17) (xy 180.34 90.17) (xy 180.34 93.98) (xy 177.8 93.98) (xy 177.8 99.06)
   (xy 173.99 99.06) (xy 173.99 102.87) (xy 170.18 102.87) (xy 170.18 105.41) (xy 173.99 105.41) (xy 173.99 111.76) (xy 177.8 111.76)
   (xy 177.8 116.84) (xy 180.34 116.84) (xy 180.34 121.92) (xy 182.88 121.92) (xy 182.88 124.46) (xy 179.07 124.46) (xy 179.07 123.19)
   (xy 176.53 123.19) (xy 176.53 120.65) (xy 172.72 120.65) (xy 172.72 118.11) (xy 156.21 118.11) (xy 156.21 115.57) (xy 152.4 115.57)
   (xy 152.4 111.76) (xy 140.97 111.76) (xy 140.97 118.11) (xy 137.16 118.11) (xy 137.16 121.92) (xy 129.54 121.92) (xy 129.54 124.46)
   (xy 120.65 124.46) (xy 120.65 125.73) (xy 118.11 125.73) (xy 118.11 118.11) (xy 114.3 118.11) (xy 114.3 107.95) (xy 116.84 107.95)
   (xy 116.84 104.14) (xy 118.11 104.14) (xy 118.11 96.52) (xy 115.57 96.52) (xy 115.57 93.98) (xy 109.22 93.98) (xy 109.22 90.17)
   (xy 107.95 90.17) (xy 107.95 82.55) (xy 105.41 82.55) (xy 105.41 74.93) (xy 104.14 74.93))
  (stroke (width 0.05) (type solid)) (fill no) (layer "Edge.Cuts"))
 (segment (start 176.075 80.34) (end 176.91 80.34) (width 0.2) (layer "F.Cu") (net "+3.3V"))
 (segment (start 158.1756 99.7982) (end 160.2121 97.7617) (width 0.2) (layer "B.Cu") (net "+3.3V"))
 (segment (start 176.075 80.34) (end 173.4144 83.0006) (width 0.2) (layer "B.Cu") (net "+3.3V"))
 (segment (start 147.7329 71.0581) (end 148.0656 71.0581) (width 0.2) (layer "B.Cu") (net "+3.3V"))
 (segment (start 161.0049 102.8566) (end 159.3498 102.8566) (width 0.2) (layer "B.Cu") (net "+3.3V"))
 (segment (start 146.7877 69.825) (end 146.7877 70.1129) (width 0.2) (layer "B.Cu") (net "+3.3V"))
 (segment (start 148.0656 71.0581) (end 148.1485 70.9752) (width 0.2) (layer "B.Cu") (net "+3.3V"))
 (segment (start 148.1485 70.9752) (end 151.3218 70.9752) (width 0.2) (layer "B.Cu") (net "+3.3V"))
 (segment (start 159.4166 79.07) (end 169.4838 79.07) (width 0.2) (layer "B.Cu") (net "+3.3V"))
 (segment (start 142.96 59.08) (end 142.96 64) (width 0.2) (layer "B.Cu") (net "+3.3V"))
 (segment (start 159.3498 101.3052) (end 158.1756 100.131) (width 0.2) (layer "B.Cu") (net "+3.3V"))
 (segment (start 145.636 69.825) (end 146.7877 69.825) (width 0.2) (layer "B.Cu") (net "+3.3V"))
 (segment (start 142.96 65.9973) (end 142.96 64) (width 0.2) (layer "B.Cu") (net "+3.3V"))
 (segment (start 173.4144 90.4471) (end 161.0049 102.8566) (width 0.2) (layer "B.Cu") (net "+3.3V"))
 (segment (start 169.4838 79.07) (end 173.4144 83.0006) (width 0.2) (layer "B.Cu") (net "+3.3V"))
 (segment (start 160.2121 97.7617) (end 160.5 97.7617) (width 0.2) (layer "B.Cu") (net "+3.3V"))
 (segment (start 141.88 58) (end 142.96 59.08) (width 0.2) (layer "B.Cu") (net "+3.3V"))
 (segment (start 145.636 69.825) (end 145.636 68.6733) (width 0.2) (layer "B.Cu") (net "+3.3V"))
 (segment (start 159.3498 102.8566) (end 159.3498 101.3052) (width 0.2) (layer "B.Cu") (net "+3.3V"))
 (segment (start 160.5 96.61) (end 160.5 97.7617) (width 0.2) (layer "B.Cu") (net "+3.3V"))
 (segment (start 173.4144 83.0006) (end 173.4144 90.4471) (width 0.2) (layer "B.Cu") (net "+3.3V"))
 (segment (start 158.1756 100.131) (end 158.1756 99.7982) (width 0.2) (layer "B.Cu") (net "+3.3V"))
 (segment (start 146.7877 70.1129) (end 147.7329 71.0581) (width 0.2) (layer "B.Cu") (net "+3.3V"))
 (segment (start 145.636 68.6733) (end 142.96 65.9973) (width 0.2) (layer "B.Cu") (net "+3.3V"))
 (segment (start 151.3218 70.9752) (end 159.4166 79.07) (width 0.2) (layer "B.Cu") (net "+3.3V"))
 (segment (start 157.7025 101.9475) (end 160.5 99.15) (width 0.2) (layer "F.Cu") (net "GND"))
 (segment (start 144.1816 74.9711) (end 122.6789 74.9711) (width 0.2) (layer "F.Cu") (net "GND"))
 (segment (start 122.6789 74.9711) (end 117.69 79.96) (width 0.2) (layer "F.Cu") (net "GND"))
 (segment (start 176.075 77.8) (end 171.3251 73.0501) (width 0.2) (layer "F.Cu") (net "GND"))
 (segment (start 148.176 69.825) (end 149.3277 69.825) (width 0.2) (layer "F.Cu") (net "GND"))
 (segment (start 125.69 102.96) (end 126.7025 101.9475) (width 0.2) (layer "F.Cu") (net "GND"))
 (segment (start 176.075 77.8) (end 176.91 77.8) (width 0.2) (layer "F.Cu") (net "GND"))
 (segment (start 149.3277 69.825) (end 144.1816 74.9711) (width 0.2) (layer "F.Cu") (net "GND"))
 (segment (start 152.5528 73.0501) (end 149.3277 69.825) (width 0.2) (layer "F.Cu") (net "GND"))
 (segment (start 126.7025 101.9475) (end 157.7025 101.9475) (width 0.2) (layer "F.Cu") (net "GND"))
 (segment (start 171.3251 73.0501) (end 152.5528 73.0501) (width 0.2) (layer "F.Cu") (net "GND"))
 (segment (start 148.176 68.6733) (end 150.58 66.2693) (width 0.2) (layer "B.Cu") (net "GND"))
 (segment (start 150.58 66.2693) (end 150.58 64) (width 0.2) (layer "B.Cu") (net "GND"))
 (segment (start 118.5686 95.8386) (end 125.69 102.96) (width 0.2) (layer "B.Cu") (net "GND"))
 (segment (start 118.5686 80.8386) (end 118.5686 95.8386) (width 0.2) (layer "B.Cu") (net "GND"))
 (segment (start 148.176 69.825) (end 148.176 68.6733) (width 0.2) (layer "B.Cu") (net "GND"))
 (segment (start 117.69 79.96) (end 118.5686 80.8386) (width 0.2) (layer "B.Cu") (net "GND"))
 (segment (start 160.835 85.42) (end 160 85.42) (width 0.2) (layer "F.Cu") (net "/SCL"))
 (segment (start 160.835 85.42) (end 162.56 87.145) (width 0.2) (layer "B.Cu") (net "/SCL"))
 (segment (start 160.835 85.42) (end 159.5742 85.42) (width 0.2) (layer "B.Cu") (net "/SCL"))
 (segment (start 162.56 99.63) (end 160.5 101.69) (width 0.2) (layer "B.Cu") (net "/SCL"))
 (segment (start 143.096 69.825) (end 144.2477 69.825) (width 0.2) (layer "B.Cu") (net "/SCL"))
 (segment (start 159.5742 85.42) (end 144.2477 70.0935) (width 0.2) (layer "B.Cu") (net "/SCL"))
 (segment (start 162.56 87.145) (end 162.56 99.63) (width 0.2) (layer "B.Cu") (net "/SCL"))
 (segment (start 144.2477 70.0935) (end 144.2477 69.825) (width 0.2) (layer "B.Cu") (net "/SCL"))
 (segment (start 160.835 87.96) (end 160 87.96) (width 0.2) (layer "F.Cu") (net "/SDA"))
 (segment (start 158.7805 87.96) (end 158.7805 98.0886) (width 0.2) (layer "B.Cu") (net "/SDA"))
 (segment (start 158.7805 98.0886) (end 157.7234 99.1457) (width 0.2) (layer "B.Cu") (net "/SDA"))
 (segment (start 160.0007 104.23) (end 160.5 104.23) (width 0.2) (layer "B.Cu") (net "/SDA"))
 (segment (start 158.7805 87.96) (end 160.835 87.96) (width 0.2) (layer "B.Cu") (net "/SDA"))
 (segment (start 157.7234 99.1457) (end 157.7234 101.9527) (width 0.2) (layer "B.Cu") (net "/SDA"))
 (segment (start 155.6905 83.7) (end 158.7805 86.79) (width 0.2) (layer "B.Cu") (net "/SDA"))
 (segment (start 157.7234 101.9527) (end 160.0007 104.23) (width 0.2) (layer "B.Cu") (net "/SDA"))
 (segment (start 158.7805 86.79) (end 158.7805 87.96) (width 0.2) (layer "B.Cu") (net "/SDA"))
 (segment (start 140.556 70.9752) (end 142.9657 70.9752) (width 0.2) (layer "B.Cu") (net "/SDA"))
 (segment (start 142.9657 70.9752) (end 155.6905 83.7) (width 0.2) (layer "B.Cu") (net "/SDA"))
 (segment (start 140.556 69.825) (end 140.556 70.9752) (width 0.2) (layer "B.Cu") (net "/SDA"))
 (segment (start 142.46 100.42) (end 132.04 100.42) (width 0.2) (layer "F.Cu") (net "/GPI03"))
 (segment (start 160 82.88) (end 142.46 100.42) (width 0.2) (layer "F.Cu") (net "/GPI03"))
 (segment (start 160.835 82.88) (end 160 82.88) (width 0.2) (layer "F.Cu") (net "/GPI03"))
 (segment (start 160.835 77.8) (end 160 77.8) (width 0.2) (layer "F.Cu") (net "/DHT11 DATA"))
 (segment (start 159.2999 76.2649) (end 159.2999 67.7999) (width 0.2) (layer "B.Cu") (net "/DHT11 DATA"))
 (segment (start 149.5 58) (end 145.5 62) (width 0.2) (layer "B.Cu") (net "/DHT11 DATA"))
 (segment (start 159.2999 67.7999) (end 149.5 58) (width 0.2) (layer "B.Cu") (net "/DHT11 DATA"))
 (segment (start 145.5 62) (end 145.5 64) (width 0.2) (layer "B.Cu") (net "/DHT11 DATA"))
 (segment (start 160.835 77.8) (end 159.2999 76.2649) (width 0.2) (layer "B.Cu") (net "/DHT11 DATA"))
 (segment (start 160 80.34) (end 126.96 80.34) (width 0.2) (layer "F.Cu") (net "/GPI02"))
 (segment (start 160.835 80.34) (end 160 80.34) (width 0.2) (layer "F.Cu") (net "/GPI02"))
 (segment (start 126.96 80.34) (end 124.04 77.42) (width 0.2) (layer "F.Cu") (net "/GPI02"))
 (segment (start 160.835 75.26) (end 160 75.26) (width 0.2) (layer "F.Cu") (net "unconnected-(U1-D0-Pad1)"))
 (segment (start 160.835 90.5) (end 160 90.5) (width 0.2) (layer "F.Cu") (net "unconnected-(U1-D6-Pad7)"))
 (segment (start 176.075 90.5) (end 176.91 90.5) (width 0.2) (layer "F.Cu") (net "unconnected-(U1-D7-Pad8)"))
 (segment (start 176.075 87.96) (end 176.91 87.96) (width 0.2) (layer "F.Cu") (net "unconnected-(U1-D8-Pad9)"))
 (segment (start 176.075 85.42) (end 176.91 85.42) (width 0.2) (layer "F.Cu") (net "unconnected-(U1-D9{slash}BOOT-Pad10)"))
 (segment (start 176.075 82.88) (end 176.91 82.88) (width 0.2) (layer "F.Cu") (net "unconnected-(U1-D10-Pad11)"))
 (segment (start 176.075 75.26) (end 176.91 75.26) (width 0.2) (layer "F.Cu") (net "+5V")))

